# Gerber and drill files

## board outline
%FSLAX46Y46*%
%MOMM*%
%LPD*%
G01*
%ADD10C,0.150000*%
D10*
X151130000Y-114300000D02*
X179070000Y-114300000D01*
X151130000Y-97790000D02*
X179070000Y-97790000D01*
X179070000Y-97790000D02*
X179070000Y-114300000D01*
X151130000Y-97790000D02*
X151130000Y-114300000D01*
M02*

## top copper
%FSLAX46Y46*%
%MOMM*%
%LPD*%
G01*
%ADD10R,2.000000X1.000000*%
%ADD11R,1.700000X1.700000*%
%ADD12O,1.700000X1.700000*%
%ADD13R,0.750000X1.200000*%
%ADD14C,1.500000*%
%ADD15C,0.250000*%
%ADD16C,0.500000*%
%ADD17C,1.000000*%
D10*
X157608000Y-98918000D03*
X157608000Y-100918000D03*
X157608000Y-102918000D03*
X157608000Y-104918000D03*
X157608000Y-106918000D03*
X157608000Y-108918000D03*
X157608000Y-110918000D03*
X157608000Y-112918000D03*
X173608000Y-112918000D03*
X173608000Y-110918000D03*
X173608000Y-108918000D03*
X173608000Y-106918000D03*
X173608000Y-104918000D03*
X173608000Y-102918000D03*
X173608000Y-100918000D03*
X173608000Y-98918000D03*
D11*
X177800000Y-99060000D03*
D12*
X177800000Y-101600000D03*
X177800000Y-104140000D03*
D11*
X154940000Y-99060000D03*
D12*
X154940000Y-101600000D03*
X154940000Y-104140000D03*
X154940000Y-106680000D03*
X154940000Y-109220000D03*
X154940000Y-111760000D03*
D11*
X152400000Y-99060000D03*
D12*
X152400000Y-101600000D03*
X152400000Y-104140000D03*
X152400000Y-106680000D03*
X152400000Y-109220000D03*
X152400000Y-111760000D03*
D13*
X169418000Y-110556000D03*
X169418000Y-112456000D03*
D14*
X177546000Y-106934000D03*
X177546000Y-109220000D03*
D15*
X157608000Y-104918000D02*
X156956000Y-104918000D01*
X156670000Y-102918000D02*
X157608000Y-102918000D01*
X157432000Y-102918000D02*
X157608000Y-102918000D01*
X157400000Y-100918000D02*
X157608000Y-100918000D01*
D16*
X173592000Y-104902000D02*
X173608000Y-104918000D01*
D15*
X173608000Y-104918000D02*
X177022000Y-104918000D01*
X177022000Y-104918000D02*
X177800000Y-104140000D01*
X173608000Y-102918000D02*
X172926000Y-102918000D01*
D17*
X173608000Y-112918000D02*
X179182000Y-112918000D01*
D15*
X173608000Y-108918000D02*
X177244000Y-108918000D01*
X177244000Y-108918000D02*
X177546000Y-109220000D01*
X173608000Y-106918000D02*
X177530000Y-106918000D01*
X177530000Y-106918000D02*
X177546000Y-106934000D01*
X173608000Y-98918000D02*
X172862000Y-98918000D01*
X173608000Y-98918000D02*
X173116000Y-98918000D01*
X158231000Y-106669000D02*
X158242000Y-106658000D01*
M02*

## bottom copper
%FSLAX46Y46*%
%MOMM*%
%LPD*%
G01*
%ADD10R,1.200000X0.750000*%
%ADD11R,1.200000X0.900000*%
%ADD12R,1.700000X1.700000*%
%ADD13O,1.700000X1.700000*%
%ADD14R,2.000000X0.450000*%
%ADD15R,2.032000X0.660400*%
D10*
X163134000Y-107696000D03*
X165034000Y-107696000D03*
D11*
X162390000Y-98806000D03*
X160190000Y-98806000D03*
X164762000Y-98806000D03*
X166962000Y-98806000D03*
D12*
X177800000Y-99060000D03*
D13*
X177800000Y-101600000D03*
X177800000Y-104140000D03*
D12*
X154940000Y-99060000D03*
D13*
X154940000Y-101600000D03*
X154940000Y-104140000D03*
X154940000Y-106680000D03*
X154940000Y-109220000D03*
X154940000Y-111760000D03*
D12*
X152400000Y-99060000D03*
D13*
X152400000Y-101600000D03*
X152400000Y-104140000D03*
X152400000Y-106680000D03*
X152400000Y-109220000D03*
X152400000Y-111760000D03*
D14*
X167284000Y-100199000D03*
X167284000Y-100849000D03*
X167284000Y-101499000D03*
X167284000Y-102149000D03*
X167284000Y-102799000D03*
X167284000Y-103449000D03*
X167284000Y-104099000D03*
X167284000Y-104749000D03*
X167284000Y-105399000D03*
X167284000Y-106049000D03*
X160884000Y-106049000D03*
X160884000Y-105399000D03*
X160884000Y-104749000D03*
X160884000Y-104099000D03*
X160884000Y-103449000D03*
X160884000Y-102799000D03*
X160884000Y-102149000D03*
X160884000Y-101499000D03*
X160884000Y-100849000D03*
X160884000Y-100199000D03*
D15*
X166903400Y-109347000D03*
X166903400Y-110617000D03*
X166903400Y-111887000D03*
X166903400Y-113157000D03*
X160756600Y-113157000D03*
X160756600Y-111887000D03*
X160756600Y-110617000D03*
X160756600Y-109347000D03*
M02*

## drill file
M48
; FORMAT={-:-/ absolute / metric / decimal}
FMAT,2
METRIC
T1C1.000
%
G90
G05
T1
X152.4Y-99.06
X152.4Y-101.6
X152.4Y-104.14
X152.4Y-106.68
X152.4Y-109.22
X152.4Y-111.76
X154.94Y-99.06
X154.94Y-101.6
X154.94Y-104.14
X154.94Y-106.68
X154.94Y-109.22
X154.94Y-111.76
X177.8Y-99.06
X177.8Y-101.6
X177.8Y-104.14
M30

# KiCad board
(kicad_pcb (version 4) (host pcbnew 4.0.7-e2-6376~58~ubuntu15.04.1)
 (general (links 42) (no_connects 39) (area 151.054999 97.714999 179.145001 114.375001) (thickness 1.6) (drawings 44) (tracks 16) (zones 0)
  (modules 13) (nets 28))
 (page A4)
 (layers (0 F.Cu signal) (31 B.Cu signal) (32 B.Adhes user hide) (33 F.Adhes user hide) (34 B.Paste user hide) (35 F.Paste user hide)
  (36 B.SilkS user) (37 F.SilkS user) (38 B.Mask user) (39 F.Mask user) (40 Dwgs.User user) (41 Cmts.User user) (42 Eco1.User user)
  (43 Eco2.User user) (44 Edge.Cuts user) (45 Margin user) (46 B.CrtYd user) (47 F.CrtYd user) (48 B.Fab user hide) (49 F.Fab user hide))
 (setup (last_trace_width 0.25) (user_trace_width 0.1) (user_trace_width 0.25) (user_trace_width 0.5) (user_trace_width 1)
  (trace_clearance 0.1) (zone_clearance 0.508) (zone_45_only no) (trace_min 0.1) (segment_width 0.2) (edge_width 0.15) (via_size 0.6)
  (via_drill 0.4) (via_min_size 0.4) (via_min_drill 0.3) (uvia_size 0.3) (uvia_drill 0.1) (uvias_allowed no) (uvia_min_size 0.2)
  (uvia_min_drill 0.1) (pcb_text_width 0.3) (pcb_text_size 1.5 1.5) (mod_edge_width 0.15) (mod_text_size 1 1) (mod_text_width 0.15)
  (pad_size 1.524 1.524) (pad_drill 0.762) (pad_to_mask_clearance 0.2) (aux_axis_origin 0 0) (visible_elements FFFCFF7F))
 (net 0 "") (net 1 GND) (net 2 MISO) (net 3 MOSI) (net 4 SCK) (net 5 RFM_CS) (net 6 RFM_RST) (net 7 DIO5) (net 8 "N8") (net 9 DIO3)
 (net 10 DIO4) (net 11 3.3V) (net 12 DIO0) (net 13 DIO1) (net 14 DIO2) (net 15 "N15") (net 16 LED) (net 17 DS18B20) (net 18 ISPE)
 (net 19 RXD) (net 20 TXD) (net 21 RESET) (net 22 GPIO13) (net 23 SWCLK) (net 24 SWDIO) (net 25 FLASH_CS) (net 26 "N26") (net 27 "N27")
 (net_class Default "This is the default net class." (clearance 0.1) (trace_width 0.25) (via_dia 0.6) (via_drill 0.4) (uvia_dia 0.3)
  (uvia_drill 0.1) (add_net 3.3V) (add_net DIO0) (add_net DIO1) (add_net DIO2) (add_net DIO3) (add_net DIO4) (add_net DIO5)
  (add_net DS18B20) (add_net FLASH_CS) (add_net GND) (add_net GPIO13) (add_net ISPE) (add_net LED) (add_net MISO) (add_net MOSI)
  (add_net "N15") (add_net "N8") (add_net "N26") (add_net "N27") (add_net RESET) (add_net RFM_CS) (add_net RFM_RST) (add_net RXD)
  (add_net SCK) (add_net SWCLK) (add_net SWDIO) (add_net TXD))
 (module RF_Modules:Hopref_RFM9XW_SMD (layer F.Cu) (at 165.608 105.918)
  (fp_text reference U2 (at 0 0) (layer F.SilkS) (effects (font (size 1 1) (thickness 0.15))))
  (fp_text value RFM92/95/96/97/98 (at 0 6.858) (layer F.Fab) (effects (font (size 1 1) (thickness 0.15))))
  (pad 1 smd rect (at -8 -7) (size 2 1) (layers F.Cu F.Paste F.Mask) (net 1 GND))
  (pad 2 smd rect (at -8 -5) (size 2 1) (layers F.Cu F.Paste F.Mask) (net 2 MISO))
  (pad 3 smd rect (at -8 -3) (size 2 1) (layers F.Cu F.Paste F.Mask) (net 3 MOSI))
  (pad 4 smd rect (at -8 -1) (size 2 1) (layers F.Cu F.Paste F.Mask) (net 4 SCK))
  (pad 5 smd rect (at -8 1) (size 2 1) (layers F.Cu F.Paste F.Mask) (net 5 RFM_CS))
  (pad 6 smd rect (at -8 3) (size 2 1) (layers F.Cu F.Paste F.Mask) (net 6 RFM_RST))
  (pad 7 smd rect (at -8 5) (size 2 1) (layers F.Cu F.Paste F.Mask) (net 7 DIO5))
  (pad 8 smd rect (at -8 7) (size 2 1) (layers F.Cu F.Paste F.Mask) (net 1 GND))
  (pad 9 smd rect (at 8 7) (size 2 1) (layers F.Cu F.Paste F.Mask) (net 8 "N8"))
  (pad 10 smd rect (at 8 5) (size 2 1) (layers F.Cu F.Paste F.Mask) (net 1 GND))
  (pad 11 smd rect (at 8 3) (size 2 1) (layers F.Cu F.Paste F.Mask) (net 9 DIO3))
  (pad 12 smd rect (at 8 1) (size 2 1) (layers F.Cu F.Paste F.Mask) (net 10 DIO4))
  (pad 13 smd rect (at 8 -1) (size 2 1) (layers F.Cu F.Paste F.Mask) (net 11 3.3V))
  (pad 14 smd rect (at 8 -3) (size 2 1) (layers F.Cu F.Paste F.Mask) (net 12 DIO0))
  (pad 15 smd rect (at 8 -5) (size 2 1) (layers F.Cu F.Paste F.Mask) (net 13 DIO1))
  (pad 16 smd rect (at 8 -7) (size 2 1) (layers F.Cu F.Paste F.Mask) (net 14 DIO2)))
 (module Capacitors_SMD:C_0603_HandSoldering (layer B.Cu) (at 164.084 107.696)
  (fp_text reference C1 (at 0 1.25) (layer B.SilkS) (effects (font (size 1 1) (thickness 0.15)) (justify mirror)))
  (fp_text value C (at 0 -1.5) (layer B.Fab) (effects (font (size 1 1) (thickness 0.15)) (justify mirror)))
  (pad 1 smd rect (at -0.95 0) (size 1.2 0.75) (layers B.Cu B.Paste B.Mask) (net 11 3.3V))
  (pad 2 smd rect (at 0.95 0) (size 1.2 0.75) (layers B.Cu B.Paste B.Mask) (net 1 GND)))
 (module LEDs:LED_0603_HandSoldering (layer B.Cu) (at 161.29 98.806 180)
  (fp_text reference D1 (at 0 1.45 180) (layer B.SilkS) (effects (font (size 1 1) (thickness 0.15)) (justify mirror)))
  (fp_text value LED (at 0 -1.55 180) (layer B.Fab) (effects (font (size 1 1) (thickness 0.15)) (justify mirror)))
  (pad 1 smd rect (at -1.1 0 180) (size 1.2 0.9) (layers B.Cu B.Paste B.Mask) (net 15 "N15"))
  (pad 2 smd rect (at 1.1 0 180) (size 1.2 0.9) (layers B.Cu B.Paste B.Mask) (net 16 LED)))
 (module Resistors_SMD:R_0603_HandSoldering (layer B.Cu) (at 165.862 98.806)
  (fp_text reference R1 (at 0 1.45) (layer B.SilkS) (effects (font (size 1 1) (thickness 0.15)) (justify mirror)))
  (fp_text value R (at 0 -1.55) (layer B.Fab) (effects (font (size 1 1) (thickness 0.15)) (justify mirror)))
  (pad 1 smd rect (at -1.1 0) (size 1.2 0.9) (layers B.Cu B.Paste B.Mask) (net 1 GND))
  (pad 2 smd rect (at 1.1 0) (size 1.2 0.9) (layers B.Cu B.Paste B.Mask) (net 15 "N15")))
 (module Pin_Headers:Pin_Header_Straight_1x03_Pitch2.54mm (layer F.Cu) (at 177.8 99.06)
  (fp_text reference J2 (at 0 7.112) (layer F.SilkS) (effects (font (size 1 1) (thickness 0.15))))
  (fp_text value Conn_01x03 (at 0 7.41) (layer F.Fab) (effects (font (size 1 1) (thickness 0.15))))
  (pad 1 thru_hole rect (at 0 0) (size 1.7 1.7) (drill 1) (layers *.Cu *.Mask) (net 1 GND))
  (pad 2 thru_hole oval (at 0 2.54) (size 1.7 1.7) (drill 1) (layers *.Cu *.Mask) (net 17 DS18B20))
  (pad 3 thru_hole oval (at 0 5.08) (size 1.7 1.7) (drill 1) (layers *.Cu *.Mask) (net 11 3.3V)))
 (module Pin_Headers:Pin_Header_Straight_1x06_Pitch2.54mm (layer F.Cu) (at 154.94 99.06)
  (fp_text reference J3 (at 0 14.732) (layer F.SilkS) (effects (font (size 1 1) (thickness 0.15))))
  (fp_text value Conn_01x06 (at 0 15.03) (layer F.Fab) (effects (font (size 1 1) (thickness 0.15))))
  (pad 1 thru_hole rect (at 0 0) (size 1.7 1.7) (drill 1) (layers *.Cu *.Mask) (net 1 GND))
  (pad 2 thru_hole oval (at 0 2.54) (size 1.7 1.7) (drill 1) (layers *.Cu *.Mask) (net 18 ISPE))
  (pad 3 thru_hole oval (at 0 5.08) (size 1.7 1.7) (drill 1) (layers *.Cu *.Mask) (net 11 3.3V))
  (pad 4 thru_hole oval (at 0 7.62) (size 1.7 1.7) (drill 1) (layers *.Cu *.Mask) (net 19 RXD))
  (pad 5 thru_hole oval (at 0 10.16) (size 1.7 1.7) (drill 1) (layers *.Cu *.Mask) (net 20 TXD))
  (pad 6 thru_hole oval (at 0 12.7) (size 1.7 1.7) (drill 1) (layers *.Cu *.Mask) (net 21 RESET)))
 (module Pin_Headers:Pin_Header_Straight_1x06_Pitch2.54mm (layer F.Cu) (at 152.4 99.06)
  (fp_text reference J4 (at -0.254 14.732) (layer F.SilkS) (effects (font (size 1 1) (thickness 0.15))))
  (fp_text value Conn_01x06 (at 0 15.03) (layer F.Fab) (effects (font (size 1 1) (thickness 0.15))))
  (pad 1 thru_hole rect (at 0 0) (size 1.7 1.7) (drill 1) (layers *.Cu *.Mask) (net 1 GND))
  (pad 2 thru_hole oval (at 0 2.54) (size 1.7 1.7) (drill 1) (layers *.Cu *.Mask) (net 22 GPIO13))
  (pad 3 thru_hole oval (at 0 5.08) (size 1.7 1.7) (drill 1) (layers *.Cu *.Mask) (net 11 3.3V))
  (pad 4 thru_hole oval (at 0 7.62) (size 1.7 1.7) (drill 1) (layers *.Cu *.Mask) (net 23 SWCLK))
  (pad 5 thru_hole oval (at 0 10.16) (size 1.7 1.7) (drill 1) (layers *.Cu *.Mask) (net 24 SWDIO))
  (pad 6 thru_hole oval (at 0 12.7) (size 1.7 1.7) (drill 1) (layers *.Cu *.Mask) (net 21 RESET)))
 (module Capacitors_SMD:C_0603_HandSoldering (layer F.Cu) (at 169.418 111.506 270)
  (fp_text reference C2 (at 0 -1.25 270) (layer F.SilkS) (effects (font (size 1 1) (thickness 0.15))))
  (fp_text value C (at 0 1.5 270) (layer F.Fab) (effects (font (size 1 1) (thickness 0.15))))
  (pad 1 smd rect (at -0.95 0 270) (size 1.2 0.75) (layers F.Cu F.Paste F.Mask) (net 11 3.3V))
  (pad 2 smd rect (at 0.95 0 270) (size 1.2 0.75) (layers F.Cu F.Paste F.Mask) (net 1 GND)))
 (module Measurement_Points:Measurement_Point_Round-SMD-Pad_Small (layer F.Cu) (at 177.546 106.934)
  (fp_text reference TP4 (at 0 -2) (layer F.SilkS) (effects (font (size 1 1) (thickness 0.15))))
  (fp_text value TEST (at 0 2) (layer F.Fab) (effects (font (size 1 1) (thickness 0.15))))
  (pad 1 smd circle (at 0 0) (size 1.5 1.5) (layers F.Cu F.Mask) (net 10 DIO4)))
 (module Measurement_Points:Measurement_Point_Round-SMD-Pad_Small (layer F.Cu) (at 177.546 109.22)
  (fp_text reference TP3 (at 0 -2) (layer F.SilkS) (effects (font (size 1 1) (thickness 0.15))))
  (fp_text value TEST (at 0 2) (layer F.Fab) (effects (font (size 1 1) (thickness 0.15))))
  (pad 1 smd circle (at 0 0) (size 1.5 1.5) (layers F.Cu F.Mask) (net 9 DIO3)))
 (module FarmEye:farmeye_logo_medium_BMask (layer F.Cu) (at 173.736 107.696 90)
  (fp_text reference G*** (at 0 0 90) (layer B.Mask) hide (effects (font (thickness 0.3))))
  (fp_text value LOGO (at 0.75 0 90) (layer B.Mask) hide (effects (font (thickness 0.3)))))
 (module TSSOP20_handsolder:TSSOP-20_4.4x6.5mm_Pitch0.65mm (layer B.Cu) (at 164.084 103.124 180)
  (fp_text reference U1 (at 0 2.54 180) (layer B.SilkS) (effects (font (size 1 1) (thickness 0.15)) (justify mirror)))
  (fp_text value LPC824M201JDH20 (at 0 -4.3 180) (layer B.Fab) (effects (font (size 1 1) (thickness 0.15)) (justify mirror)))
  (pad 1 smd rect (at -3.2 2.925 180) (size 2 0.45) (layers B.Cu B.Paste B.Mask) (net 12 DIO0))
  (pad 2 smd rect (at -3.2 2.275 180) (size 2 0.45) (layers B.Cu B.Paste B.Mask) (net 16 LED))
  (pad 3 smd rect (at -3.2 1.625 180) (size 2 0.45) (layers B.Cu B.Paste B.Mask) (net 22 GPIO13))
  (pad 4 smd rect (at -3.2 0.975 180) (size 2 0.45) (layers B.Cu B.Paste B.Mask) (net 18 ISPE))
  (pad 5 smd rect (at -3.2 0.325 180) (size 2 0.45) (layers B.Cu B.Paste B.Mask) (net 21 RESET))
  (pad 6 smd rect (at -3.2 -0.325 180) (size 2 0.45) (layers B.Cu B.Paste B.Mask) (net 20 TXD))
  (pad 7 smd rect (at -3.2 -0.975 180) (size 2 0.45) (layers B.Cu B.Paste B.Mask) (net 23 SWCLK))
  (pad 8 smd rect (at -3.2 -1.625 180) (size 2 0.45) (layers B.Cu B.Paste B.Mask) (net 24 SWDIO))
  (pad 9 smd rect (at -3.2 -2.275 180) (size 2 0.45) (layers B.Cu B.Paste B.Mask) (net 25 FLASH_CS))
  (pad 10 smd rect (at -3.2 -2.925 180) (size 2 0.45) (layers B.Cu B.Paste B.Mask) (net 17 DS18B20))
  (pad 11 smd rect (at 3.2 -2.925 180) (size 2 0.45) (layers B.Cu B.Paste B.Mask) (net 6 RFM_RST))
  (pad 12 smd rect (at 3.2 -2.275 180) (size 2 0.45) (layers B.Cu B.Paste B.Mask) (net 4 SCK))
  (pad 13 smd rect (at 3.2 -1.625 180) (size 2 0.45) (layers B.Cu B.Paste B.Mask) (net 3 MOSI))
  (pad 14 smd rect (at 3.2 -0.975 180) (size 2 0.45) (layers B.Cu B.Paste B.Mask) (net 2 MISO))
  (pad 15 smd rect (at 3.2 -0.325 180) (size 2 0.45) (layers B.Cu B.Paste B.Mask) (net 11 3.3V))
  (pad 16 smd rect (at 3.2 0.325 180) (size 2 0.45) (layers B.Cu B.Paste B.Mask) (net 1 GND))
  (pad 17 smd rect (at 3.2 0.975 180) (size 2 0.45) (layers B.Cu B.Paste B.Mask) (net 1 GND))
  (pad 18 smd rect (at 3.2 1.625 180) (size 2 0.45) (layers B.Cu B.Paste B.Mask) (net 11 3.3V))
  (pad 19 smd rect (at 3.2 2.275 180) (size 2 0.45) (layers B.Cu B.Paste B.Mask) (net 19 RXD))
  (pad 20 smd rect (at 3.2 2.925 180) (size 2 0.45) (layers B.Cu B.Paste B.Mask) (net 5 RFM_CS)))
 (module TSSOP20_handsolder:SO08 (layer B.Cu) (at 163.83 111.252 270)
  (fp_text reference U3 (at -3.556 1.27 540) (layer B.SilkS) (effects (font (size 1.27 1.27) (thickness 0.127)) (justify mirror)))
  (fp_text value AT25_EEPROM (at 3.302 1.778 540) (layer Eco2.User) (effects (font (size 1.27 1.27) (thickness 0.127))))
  (pad 1 smd rect (at -1.905 -3.0734 270) (size 0.6604 2.032) (layers B.Cu B.Paste B.Mask) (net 25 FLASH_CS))
  (pad 2 smd rect (at -0.635 -3.0734 270) (size 0.6604 2.032) (layers B.Cu B.Paste B.Mask) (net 2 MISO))
  (pad 3 smd rect (at 0.635 -3.0734 270) (size 0.6604 2.032) (layers B.Cu B.Paste B.Mask) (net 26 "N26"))
  (pad 4 smd rect (at 1.905 -3.0734 270) (size 0.6604 2.032) (layers B.Cu B.Paste B.Mask) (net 1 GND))
  (pad 5 smd rect (at 1.905 3.0734 270) (size 0.6604 2.032) (layers B.Cu B.Paste B.Mask) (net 3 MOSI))
  (pad 6 smd rect (at 0.635 3.0734 270) (size 0.6604 2.032) (layers B.Cu B.Paste B.Mask) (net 4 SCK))
  (pad 7 smd rect (at -0.635 3.0734 270) (size 0.6604 2.032) (layers B.Cu B.Paste B.Mask) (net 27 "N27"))
  (pad 8 smd rect (at -1.905 3.0734 270) (size 0.6604 2.032) (layers B.Cu B.Paste B.Mask) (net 11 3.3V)))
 (gr_line (start 151.13 114.3) (end 179.07 114.3) (angle 90) (layer Edge.Cuts) (width 0.15))
 (gr_line (start 151.13 97.79) (end 179.07 97.79) (angle 90) (layer Edge.Cuts) (width 0.15))
 (gr_line (start 179.07 97.79) (end 179.07 114.3) (angle 90) (layer Edge.Cuts) (width 0.15))
 (gr_line (start 151.13 97.79) (end 151.13 114.3) (angle 90) (layer Edge.Cuts) (width 0.15))
 (segment (start 157.608 104.918) (end 156.956 104.918) (width 0.25) (layer F.Cu) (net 4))
 (segment (start 156.67 102.918) (end 157.608 102.918) (width 0.25) (layer F.Cu) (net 3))
 (segment (start 157.432 102.918) (end 157.608 102.918) (width 0.25) (layer F.Cu) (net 3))
 (segment (start 157.4 100.918) (end 157.608 100.918) (width 0.25) (layer F.Cu) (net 2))
 (segment (start 173.592 104.902) (end 173.608 104.918) (width 0.5) (layer F.Cu) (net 11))
 (segment (start 173.608 104.918) (end 177.022 104.918) (width 0.25) (layer F.Cu) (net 11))
 (segment (start 177.022 104.918) (end 177.8 104.14) (width 0.25) (layer F.Cu) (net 11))
 (segment (start 173.608 102.918) (end 172.926 102.918) (width 0.25) (layer F.Cu) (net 12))
 (segment (start 173.608 112.918) (end 179.182 112.918) (width 1) (layer F.Cu) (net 8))
 (segment (start 173.608 108.918) (end 177.244 108.918) (width 0.25) (layer F.Cu) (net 9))
 (segment (start 177.244 108.918) (end 177.546 109.22) (width 0.25) (layer F.Cu) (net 9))
 (segment (start 173.608 106.918) (end 177.53 106.918) (width 0.25) (layer F.Cu) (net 10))
 (segment (start 177.53 106.918) (end 177.546 106.934) (width 0.25) (layer F.Cu) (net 10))
 (segment (start 173.608 98.918) (end 172.862 98.918) (width 0.25) (layer F.Cu) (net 14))
 (segment (start 173.608 98.918) (end 173.116 98.918) (width 0.25) (layer F.Cu) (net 14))
 (segment (start 158.231 106.669) (end 158.242 106.658) (width 0.25) (layer F.Cu) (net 5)))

